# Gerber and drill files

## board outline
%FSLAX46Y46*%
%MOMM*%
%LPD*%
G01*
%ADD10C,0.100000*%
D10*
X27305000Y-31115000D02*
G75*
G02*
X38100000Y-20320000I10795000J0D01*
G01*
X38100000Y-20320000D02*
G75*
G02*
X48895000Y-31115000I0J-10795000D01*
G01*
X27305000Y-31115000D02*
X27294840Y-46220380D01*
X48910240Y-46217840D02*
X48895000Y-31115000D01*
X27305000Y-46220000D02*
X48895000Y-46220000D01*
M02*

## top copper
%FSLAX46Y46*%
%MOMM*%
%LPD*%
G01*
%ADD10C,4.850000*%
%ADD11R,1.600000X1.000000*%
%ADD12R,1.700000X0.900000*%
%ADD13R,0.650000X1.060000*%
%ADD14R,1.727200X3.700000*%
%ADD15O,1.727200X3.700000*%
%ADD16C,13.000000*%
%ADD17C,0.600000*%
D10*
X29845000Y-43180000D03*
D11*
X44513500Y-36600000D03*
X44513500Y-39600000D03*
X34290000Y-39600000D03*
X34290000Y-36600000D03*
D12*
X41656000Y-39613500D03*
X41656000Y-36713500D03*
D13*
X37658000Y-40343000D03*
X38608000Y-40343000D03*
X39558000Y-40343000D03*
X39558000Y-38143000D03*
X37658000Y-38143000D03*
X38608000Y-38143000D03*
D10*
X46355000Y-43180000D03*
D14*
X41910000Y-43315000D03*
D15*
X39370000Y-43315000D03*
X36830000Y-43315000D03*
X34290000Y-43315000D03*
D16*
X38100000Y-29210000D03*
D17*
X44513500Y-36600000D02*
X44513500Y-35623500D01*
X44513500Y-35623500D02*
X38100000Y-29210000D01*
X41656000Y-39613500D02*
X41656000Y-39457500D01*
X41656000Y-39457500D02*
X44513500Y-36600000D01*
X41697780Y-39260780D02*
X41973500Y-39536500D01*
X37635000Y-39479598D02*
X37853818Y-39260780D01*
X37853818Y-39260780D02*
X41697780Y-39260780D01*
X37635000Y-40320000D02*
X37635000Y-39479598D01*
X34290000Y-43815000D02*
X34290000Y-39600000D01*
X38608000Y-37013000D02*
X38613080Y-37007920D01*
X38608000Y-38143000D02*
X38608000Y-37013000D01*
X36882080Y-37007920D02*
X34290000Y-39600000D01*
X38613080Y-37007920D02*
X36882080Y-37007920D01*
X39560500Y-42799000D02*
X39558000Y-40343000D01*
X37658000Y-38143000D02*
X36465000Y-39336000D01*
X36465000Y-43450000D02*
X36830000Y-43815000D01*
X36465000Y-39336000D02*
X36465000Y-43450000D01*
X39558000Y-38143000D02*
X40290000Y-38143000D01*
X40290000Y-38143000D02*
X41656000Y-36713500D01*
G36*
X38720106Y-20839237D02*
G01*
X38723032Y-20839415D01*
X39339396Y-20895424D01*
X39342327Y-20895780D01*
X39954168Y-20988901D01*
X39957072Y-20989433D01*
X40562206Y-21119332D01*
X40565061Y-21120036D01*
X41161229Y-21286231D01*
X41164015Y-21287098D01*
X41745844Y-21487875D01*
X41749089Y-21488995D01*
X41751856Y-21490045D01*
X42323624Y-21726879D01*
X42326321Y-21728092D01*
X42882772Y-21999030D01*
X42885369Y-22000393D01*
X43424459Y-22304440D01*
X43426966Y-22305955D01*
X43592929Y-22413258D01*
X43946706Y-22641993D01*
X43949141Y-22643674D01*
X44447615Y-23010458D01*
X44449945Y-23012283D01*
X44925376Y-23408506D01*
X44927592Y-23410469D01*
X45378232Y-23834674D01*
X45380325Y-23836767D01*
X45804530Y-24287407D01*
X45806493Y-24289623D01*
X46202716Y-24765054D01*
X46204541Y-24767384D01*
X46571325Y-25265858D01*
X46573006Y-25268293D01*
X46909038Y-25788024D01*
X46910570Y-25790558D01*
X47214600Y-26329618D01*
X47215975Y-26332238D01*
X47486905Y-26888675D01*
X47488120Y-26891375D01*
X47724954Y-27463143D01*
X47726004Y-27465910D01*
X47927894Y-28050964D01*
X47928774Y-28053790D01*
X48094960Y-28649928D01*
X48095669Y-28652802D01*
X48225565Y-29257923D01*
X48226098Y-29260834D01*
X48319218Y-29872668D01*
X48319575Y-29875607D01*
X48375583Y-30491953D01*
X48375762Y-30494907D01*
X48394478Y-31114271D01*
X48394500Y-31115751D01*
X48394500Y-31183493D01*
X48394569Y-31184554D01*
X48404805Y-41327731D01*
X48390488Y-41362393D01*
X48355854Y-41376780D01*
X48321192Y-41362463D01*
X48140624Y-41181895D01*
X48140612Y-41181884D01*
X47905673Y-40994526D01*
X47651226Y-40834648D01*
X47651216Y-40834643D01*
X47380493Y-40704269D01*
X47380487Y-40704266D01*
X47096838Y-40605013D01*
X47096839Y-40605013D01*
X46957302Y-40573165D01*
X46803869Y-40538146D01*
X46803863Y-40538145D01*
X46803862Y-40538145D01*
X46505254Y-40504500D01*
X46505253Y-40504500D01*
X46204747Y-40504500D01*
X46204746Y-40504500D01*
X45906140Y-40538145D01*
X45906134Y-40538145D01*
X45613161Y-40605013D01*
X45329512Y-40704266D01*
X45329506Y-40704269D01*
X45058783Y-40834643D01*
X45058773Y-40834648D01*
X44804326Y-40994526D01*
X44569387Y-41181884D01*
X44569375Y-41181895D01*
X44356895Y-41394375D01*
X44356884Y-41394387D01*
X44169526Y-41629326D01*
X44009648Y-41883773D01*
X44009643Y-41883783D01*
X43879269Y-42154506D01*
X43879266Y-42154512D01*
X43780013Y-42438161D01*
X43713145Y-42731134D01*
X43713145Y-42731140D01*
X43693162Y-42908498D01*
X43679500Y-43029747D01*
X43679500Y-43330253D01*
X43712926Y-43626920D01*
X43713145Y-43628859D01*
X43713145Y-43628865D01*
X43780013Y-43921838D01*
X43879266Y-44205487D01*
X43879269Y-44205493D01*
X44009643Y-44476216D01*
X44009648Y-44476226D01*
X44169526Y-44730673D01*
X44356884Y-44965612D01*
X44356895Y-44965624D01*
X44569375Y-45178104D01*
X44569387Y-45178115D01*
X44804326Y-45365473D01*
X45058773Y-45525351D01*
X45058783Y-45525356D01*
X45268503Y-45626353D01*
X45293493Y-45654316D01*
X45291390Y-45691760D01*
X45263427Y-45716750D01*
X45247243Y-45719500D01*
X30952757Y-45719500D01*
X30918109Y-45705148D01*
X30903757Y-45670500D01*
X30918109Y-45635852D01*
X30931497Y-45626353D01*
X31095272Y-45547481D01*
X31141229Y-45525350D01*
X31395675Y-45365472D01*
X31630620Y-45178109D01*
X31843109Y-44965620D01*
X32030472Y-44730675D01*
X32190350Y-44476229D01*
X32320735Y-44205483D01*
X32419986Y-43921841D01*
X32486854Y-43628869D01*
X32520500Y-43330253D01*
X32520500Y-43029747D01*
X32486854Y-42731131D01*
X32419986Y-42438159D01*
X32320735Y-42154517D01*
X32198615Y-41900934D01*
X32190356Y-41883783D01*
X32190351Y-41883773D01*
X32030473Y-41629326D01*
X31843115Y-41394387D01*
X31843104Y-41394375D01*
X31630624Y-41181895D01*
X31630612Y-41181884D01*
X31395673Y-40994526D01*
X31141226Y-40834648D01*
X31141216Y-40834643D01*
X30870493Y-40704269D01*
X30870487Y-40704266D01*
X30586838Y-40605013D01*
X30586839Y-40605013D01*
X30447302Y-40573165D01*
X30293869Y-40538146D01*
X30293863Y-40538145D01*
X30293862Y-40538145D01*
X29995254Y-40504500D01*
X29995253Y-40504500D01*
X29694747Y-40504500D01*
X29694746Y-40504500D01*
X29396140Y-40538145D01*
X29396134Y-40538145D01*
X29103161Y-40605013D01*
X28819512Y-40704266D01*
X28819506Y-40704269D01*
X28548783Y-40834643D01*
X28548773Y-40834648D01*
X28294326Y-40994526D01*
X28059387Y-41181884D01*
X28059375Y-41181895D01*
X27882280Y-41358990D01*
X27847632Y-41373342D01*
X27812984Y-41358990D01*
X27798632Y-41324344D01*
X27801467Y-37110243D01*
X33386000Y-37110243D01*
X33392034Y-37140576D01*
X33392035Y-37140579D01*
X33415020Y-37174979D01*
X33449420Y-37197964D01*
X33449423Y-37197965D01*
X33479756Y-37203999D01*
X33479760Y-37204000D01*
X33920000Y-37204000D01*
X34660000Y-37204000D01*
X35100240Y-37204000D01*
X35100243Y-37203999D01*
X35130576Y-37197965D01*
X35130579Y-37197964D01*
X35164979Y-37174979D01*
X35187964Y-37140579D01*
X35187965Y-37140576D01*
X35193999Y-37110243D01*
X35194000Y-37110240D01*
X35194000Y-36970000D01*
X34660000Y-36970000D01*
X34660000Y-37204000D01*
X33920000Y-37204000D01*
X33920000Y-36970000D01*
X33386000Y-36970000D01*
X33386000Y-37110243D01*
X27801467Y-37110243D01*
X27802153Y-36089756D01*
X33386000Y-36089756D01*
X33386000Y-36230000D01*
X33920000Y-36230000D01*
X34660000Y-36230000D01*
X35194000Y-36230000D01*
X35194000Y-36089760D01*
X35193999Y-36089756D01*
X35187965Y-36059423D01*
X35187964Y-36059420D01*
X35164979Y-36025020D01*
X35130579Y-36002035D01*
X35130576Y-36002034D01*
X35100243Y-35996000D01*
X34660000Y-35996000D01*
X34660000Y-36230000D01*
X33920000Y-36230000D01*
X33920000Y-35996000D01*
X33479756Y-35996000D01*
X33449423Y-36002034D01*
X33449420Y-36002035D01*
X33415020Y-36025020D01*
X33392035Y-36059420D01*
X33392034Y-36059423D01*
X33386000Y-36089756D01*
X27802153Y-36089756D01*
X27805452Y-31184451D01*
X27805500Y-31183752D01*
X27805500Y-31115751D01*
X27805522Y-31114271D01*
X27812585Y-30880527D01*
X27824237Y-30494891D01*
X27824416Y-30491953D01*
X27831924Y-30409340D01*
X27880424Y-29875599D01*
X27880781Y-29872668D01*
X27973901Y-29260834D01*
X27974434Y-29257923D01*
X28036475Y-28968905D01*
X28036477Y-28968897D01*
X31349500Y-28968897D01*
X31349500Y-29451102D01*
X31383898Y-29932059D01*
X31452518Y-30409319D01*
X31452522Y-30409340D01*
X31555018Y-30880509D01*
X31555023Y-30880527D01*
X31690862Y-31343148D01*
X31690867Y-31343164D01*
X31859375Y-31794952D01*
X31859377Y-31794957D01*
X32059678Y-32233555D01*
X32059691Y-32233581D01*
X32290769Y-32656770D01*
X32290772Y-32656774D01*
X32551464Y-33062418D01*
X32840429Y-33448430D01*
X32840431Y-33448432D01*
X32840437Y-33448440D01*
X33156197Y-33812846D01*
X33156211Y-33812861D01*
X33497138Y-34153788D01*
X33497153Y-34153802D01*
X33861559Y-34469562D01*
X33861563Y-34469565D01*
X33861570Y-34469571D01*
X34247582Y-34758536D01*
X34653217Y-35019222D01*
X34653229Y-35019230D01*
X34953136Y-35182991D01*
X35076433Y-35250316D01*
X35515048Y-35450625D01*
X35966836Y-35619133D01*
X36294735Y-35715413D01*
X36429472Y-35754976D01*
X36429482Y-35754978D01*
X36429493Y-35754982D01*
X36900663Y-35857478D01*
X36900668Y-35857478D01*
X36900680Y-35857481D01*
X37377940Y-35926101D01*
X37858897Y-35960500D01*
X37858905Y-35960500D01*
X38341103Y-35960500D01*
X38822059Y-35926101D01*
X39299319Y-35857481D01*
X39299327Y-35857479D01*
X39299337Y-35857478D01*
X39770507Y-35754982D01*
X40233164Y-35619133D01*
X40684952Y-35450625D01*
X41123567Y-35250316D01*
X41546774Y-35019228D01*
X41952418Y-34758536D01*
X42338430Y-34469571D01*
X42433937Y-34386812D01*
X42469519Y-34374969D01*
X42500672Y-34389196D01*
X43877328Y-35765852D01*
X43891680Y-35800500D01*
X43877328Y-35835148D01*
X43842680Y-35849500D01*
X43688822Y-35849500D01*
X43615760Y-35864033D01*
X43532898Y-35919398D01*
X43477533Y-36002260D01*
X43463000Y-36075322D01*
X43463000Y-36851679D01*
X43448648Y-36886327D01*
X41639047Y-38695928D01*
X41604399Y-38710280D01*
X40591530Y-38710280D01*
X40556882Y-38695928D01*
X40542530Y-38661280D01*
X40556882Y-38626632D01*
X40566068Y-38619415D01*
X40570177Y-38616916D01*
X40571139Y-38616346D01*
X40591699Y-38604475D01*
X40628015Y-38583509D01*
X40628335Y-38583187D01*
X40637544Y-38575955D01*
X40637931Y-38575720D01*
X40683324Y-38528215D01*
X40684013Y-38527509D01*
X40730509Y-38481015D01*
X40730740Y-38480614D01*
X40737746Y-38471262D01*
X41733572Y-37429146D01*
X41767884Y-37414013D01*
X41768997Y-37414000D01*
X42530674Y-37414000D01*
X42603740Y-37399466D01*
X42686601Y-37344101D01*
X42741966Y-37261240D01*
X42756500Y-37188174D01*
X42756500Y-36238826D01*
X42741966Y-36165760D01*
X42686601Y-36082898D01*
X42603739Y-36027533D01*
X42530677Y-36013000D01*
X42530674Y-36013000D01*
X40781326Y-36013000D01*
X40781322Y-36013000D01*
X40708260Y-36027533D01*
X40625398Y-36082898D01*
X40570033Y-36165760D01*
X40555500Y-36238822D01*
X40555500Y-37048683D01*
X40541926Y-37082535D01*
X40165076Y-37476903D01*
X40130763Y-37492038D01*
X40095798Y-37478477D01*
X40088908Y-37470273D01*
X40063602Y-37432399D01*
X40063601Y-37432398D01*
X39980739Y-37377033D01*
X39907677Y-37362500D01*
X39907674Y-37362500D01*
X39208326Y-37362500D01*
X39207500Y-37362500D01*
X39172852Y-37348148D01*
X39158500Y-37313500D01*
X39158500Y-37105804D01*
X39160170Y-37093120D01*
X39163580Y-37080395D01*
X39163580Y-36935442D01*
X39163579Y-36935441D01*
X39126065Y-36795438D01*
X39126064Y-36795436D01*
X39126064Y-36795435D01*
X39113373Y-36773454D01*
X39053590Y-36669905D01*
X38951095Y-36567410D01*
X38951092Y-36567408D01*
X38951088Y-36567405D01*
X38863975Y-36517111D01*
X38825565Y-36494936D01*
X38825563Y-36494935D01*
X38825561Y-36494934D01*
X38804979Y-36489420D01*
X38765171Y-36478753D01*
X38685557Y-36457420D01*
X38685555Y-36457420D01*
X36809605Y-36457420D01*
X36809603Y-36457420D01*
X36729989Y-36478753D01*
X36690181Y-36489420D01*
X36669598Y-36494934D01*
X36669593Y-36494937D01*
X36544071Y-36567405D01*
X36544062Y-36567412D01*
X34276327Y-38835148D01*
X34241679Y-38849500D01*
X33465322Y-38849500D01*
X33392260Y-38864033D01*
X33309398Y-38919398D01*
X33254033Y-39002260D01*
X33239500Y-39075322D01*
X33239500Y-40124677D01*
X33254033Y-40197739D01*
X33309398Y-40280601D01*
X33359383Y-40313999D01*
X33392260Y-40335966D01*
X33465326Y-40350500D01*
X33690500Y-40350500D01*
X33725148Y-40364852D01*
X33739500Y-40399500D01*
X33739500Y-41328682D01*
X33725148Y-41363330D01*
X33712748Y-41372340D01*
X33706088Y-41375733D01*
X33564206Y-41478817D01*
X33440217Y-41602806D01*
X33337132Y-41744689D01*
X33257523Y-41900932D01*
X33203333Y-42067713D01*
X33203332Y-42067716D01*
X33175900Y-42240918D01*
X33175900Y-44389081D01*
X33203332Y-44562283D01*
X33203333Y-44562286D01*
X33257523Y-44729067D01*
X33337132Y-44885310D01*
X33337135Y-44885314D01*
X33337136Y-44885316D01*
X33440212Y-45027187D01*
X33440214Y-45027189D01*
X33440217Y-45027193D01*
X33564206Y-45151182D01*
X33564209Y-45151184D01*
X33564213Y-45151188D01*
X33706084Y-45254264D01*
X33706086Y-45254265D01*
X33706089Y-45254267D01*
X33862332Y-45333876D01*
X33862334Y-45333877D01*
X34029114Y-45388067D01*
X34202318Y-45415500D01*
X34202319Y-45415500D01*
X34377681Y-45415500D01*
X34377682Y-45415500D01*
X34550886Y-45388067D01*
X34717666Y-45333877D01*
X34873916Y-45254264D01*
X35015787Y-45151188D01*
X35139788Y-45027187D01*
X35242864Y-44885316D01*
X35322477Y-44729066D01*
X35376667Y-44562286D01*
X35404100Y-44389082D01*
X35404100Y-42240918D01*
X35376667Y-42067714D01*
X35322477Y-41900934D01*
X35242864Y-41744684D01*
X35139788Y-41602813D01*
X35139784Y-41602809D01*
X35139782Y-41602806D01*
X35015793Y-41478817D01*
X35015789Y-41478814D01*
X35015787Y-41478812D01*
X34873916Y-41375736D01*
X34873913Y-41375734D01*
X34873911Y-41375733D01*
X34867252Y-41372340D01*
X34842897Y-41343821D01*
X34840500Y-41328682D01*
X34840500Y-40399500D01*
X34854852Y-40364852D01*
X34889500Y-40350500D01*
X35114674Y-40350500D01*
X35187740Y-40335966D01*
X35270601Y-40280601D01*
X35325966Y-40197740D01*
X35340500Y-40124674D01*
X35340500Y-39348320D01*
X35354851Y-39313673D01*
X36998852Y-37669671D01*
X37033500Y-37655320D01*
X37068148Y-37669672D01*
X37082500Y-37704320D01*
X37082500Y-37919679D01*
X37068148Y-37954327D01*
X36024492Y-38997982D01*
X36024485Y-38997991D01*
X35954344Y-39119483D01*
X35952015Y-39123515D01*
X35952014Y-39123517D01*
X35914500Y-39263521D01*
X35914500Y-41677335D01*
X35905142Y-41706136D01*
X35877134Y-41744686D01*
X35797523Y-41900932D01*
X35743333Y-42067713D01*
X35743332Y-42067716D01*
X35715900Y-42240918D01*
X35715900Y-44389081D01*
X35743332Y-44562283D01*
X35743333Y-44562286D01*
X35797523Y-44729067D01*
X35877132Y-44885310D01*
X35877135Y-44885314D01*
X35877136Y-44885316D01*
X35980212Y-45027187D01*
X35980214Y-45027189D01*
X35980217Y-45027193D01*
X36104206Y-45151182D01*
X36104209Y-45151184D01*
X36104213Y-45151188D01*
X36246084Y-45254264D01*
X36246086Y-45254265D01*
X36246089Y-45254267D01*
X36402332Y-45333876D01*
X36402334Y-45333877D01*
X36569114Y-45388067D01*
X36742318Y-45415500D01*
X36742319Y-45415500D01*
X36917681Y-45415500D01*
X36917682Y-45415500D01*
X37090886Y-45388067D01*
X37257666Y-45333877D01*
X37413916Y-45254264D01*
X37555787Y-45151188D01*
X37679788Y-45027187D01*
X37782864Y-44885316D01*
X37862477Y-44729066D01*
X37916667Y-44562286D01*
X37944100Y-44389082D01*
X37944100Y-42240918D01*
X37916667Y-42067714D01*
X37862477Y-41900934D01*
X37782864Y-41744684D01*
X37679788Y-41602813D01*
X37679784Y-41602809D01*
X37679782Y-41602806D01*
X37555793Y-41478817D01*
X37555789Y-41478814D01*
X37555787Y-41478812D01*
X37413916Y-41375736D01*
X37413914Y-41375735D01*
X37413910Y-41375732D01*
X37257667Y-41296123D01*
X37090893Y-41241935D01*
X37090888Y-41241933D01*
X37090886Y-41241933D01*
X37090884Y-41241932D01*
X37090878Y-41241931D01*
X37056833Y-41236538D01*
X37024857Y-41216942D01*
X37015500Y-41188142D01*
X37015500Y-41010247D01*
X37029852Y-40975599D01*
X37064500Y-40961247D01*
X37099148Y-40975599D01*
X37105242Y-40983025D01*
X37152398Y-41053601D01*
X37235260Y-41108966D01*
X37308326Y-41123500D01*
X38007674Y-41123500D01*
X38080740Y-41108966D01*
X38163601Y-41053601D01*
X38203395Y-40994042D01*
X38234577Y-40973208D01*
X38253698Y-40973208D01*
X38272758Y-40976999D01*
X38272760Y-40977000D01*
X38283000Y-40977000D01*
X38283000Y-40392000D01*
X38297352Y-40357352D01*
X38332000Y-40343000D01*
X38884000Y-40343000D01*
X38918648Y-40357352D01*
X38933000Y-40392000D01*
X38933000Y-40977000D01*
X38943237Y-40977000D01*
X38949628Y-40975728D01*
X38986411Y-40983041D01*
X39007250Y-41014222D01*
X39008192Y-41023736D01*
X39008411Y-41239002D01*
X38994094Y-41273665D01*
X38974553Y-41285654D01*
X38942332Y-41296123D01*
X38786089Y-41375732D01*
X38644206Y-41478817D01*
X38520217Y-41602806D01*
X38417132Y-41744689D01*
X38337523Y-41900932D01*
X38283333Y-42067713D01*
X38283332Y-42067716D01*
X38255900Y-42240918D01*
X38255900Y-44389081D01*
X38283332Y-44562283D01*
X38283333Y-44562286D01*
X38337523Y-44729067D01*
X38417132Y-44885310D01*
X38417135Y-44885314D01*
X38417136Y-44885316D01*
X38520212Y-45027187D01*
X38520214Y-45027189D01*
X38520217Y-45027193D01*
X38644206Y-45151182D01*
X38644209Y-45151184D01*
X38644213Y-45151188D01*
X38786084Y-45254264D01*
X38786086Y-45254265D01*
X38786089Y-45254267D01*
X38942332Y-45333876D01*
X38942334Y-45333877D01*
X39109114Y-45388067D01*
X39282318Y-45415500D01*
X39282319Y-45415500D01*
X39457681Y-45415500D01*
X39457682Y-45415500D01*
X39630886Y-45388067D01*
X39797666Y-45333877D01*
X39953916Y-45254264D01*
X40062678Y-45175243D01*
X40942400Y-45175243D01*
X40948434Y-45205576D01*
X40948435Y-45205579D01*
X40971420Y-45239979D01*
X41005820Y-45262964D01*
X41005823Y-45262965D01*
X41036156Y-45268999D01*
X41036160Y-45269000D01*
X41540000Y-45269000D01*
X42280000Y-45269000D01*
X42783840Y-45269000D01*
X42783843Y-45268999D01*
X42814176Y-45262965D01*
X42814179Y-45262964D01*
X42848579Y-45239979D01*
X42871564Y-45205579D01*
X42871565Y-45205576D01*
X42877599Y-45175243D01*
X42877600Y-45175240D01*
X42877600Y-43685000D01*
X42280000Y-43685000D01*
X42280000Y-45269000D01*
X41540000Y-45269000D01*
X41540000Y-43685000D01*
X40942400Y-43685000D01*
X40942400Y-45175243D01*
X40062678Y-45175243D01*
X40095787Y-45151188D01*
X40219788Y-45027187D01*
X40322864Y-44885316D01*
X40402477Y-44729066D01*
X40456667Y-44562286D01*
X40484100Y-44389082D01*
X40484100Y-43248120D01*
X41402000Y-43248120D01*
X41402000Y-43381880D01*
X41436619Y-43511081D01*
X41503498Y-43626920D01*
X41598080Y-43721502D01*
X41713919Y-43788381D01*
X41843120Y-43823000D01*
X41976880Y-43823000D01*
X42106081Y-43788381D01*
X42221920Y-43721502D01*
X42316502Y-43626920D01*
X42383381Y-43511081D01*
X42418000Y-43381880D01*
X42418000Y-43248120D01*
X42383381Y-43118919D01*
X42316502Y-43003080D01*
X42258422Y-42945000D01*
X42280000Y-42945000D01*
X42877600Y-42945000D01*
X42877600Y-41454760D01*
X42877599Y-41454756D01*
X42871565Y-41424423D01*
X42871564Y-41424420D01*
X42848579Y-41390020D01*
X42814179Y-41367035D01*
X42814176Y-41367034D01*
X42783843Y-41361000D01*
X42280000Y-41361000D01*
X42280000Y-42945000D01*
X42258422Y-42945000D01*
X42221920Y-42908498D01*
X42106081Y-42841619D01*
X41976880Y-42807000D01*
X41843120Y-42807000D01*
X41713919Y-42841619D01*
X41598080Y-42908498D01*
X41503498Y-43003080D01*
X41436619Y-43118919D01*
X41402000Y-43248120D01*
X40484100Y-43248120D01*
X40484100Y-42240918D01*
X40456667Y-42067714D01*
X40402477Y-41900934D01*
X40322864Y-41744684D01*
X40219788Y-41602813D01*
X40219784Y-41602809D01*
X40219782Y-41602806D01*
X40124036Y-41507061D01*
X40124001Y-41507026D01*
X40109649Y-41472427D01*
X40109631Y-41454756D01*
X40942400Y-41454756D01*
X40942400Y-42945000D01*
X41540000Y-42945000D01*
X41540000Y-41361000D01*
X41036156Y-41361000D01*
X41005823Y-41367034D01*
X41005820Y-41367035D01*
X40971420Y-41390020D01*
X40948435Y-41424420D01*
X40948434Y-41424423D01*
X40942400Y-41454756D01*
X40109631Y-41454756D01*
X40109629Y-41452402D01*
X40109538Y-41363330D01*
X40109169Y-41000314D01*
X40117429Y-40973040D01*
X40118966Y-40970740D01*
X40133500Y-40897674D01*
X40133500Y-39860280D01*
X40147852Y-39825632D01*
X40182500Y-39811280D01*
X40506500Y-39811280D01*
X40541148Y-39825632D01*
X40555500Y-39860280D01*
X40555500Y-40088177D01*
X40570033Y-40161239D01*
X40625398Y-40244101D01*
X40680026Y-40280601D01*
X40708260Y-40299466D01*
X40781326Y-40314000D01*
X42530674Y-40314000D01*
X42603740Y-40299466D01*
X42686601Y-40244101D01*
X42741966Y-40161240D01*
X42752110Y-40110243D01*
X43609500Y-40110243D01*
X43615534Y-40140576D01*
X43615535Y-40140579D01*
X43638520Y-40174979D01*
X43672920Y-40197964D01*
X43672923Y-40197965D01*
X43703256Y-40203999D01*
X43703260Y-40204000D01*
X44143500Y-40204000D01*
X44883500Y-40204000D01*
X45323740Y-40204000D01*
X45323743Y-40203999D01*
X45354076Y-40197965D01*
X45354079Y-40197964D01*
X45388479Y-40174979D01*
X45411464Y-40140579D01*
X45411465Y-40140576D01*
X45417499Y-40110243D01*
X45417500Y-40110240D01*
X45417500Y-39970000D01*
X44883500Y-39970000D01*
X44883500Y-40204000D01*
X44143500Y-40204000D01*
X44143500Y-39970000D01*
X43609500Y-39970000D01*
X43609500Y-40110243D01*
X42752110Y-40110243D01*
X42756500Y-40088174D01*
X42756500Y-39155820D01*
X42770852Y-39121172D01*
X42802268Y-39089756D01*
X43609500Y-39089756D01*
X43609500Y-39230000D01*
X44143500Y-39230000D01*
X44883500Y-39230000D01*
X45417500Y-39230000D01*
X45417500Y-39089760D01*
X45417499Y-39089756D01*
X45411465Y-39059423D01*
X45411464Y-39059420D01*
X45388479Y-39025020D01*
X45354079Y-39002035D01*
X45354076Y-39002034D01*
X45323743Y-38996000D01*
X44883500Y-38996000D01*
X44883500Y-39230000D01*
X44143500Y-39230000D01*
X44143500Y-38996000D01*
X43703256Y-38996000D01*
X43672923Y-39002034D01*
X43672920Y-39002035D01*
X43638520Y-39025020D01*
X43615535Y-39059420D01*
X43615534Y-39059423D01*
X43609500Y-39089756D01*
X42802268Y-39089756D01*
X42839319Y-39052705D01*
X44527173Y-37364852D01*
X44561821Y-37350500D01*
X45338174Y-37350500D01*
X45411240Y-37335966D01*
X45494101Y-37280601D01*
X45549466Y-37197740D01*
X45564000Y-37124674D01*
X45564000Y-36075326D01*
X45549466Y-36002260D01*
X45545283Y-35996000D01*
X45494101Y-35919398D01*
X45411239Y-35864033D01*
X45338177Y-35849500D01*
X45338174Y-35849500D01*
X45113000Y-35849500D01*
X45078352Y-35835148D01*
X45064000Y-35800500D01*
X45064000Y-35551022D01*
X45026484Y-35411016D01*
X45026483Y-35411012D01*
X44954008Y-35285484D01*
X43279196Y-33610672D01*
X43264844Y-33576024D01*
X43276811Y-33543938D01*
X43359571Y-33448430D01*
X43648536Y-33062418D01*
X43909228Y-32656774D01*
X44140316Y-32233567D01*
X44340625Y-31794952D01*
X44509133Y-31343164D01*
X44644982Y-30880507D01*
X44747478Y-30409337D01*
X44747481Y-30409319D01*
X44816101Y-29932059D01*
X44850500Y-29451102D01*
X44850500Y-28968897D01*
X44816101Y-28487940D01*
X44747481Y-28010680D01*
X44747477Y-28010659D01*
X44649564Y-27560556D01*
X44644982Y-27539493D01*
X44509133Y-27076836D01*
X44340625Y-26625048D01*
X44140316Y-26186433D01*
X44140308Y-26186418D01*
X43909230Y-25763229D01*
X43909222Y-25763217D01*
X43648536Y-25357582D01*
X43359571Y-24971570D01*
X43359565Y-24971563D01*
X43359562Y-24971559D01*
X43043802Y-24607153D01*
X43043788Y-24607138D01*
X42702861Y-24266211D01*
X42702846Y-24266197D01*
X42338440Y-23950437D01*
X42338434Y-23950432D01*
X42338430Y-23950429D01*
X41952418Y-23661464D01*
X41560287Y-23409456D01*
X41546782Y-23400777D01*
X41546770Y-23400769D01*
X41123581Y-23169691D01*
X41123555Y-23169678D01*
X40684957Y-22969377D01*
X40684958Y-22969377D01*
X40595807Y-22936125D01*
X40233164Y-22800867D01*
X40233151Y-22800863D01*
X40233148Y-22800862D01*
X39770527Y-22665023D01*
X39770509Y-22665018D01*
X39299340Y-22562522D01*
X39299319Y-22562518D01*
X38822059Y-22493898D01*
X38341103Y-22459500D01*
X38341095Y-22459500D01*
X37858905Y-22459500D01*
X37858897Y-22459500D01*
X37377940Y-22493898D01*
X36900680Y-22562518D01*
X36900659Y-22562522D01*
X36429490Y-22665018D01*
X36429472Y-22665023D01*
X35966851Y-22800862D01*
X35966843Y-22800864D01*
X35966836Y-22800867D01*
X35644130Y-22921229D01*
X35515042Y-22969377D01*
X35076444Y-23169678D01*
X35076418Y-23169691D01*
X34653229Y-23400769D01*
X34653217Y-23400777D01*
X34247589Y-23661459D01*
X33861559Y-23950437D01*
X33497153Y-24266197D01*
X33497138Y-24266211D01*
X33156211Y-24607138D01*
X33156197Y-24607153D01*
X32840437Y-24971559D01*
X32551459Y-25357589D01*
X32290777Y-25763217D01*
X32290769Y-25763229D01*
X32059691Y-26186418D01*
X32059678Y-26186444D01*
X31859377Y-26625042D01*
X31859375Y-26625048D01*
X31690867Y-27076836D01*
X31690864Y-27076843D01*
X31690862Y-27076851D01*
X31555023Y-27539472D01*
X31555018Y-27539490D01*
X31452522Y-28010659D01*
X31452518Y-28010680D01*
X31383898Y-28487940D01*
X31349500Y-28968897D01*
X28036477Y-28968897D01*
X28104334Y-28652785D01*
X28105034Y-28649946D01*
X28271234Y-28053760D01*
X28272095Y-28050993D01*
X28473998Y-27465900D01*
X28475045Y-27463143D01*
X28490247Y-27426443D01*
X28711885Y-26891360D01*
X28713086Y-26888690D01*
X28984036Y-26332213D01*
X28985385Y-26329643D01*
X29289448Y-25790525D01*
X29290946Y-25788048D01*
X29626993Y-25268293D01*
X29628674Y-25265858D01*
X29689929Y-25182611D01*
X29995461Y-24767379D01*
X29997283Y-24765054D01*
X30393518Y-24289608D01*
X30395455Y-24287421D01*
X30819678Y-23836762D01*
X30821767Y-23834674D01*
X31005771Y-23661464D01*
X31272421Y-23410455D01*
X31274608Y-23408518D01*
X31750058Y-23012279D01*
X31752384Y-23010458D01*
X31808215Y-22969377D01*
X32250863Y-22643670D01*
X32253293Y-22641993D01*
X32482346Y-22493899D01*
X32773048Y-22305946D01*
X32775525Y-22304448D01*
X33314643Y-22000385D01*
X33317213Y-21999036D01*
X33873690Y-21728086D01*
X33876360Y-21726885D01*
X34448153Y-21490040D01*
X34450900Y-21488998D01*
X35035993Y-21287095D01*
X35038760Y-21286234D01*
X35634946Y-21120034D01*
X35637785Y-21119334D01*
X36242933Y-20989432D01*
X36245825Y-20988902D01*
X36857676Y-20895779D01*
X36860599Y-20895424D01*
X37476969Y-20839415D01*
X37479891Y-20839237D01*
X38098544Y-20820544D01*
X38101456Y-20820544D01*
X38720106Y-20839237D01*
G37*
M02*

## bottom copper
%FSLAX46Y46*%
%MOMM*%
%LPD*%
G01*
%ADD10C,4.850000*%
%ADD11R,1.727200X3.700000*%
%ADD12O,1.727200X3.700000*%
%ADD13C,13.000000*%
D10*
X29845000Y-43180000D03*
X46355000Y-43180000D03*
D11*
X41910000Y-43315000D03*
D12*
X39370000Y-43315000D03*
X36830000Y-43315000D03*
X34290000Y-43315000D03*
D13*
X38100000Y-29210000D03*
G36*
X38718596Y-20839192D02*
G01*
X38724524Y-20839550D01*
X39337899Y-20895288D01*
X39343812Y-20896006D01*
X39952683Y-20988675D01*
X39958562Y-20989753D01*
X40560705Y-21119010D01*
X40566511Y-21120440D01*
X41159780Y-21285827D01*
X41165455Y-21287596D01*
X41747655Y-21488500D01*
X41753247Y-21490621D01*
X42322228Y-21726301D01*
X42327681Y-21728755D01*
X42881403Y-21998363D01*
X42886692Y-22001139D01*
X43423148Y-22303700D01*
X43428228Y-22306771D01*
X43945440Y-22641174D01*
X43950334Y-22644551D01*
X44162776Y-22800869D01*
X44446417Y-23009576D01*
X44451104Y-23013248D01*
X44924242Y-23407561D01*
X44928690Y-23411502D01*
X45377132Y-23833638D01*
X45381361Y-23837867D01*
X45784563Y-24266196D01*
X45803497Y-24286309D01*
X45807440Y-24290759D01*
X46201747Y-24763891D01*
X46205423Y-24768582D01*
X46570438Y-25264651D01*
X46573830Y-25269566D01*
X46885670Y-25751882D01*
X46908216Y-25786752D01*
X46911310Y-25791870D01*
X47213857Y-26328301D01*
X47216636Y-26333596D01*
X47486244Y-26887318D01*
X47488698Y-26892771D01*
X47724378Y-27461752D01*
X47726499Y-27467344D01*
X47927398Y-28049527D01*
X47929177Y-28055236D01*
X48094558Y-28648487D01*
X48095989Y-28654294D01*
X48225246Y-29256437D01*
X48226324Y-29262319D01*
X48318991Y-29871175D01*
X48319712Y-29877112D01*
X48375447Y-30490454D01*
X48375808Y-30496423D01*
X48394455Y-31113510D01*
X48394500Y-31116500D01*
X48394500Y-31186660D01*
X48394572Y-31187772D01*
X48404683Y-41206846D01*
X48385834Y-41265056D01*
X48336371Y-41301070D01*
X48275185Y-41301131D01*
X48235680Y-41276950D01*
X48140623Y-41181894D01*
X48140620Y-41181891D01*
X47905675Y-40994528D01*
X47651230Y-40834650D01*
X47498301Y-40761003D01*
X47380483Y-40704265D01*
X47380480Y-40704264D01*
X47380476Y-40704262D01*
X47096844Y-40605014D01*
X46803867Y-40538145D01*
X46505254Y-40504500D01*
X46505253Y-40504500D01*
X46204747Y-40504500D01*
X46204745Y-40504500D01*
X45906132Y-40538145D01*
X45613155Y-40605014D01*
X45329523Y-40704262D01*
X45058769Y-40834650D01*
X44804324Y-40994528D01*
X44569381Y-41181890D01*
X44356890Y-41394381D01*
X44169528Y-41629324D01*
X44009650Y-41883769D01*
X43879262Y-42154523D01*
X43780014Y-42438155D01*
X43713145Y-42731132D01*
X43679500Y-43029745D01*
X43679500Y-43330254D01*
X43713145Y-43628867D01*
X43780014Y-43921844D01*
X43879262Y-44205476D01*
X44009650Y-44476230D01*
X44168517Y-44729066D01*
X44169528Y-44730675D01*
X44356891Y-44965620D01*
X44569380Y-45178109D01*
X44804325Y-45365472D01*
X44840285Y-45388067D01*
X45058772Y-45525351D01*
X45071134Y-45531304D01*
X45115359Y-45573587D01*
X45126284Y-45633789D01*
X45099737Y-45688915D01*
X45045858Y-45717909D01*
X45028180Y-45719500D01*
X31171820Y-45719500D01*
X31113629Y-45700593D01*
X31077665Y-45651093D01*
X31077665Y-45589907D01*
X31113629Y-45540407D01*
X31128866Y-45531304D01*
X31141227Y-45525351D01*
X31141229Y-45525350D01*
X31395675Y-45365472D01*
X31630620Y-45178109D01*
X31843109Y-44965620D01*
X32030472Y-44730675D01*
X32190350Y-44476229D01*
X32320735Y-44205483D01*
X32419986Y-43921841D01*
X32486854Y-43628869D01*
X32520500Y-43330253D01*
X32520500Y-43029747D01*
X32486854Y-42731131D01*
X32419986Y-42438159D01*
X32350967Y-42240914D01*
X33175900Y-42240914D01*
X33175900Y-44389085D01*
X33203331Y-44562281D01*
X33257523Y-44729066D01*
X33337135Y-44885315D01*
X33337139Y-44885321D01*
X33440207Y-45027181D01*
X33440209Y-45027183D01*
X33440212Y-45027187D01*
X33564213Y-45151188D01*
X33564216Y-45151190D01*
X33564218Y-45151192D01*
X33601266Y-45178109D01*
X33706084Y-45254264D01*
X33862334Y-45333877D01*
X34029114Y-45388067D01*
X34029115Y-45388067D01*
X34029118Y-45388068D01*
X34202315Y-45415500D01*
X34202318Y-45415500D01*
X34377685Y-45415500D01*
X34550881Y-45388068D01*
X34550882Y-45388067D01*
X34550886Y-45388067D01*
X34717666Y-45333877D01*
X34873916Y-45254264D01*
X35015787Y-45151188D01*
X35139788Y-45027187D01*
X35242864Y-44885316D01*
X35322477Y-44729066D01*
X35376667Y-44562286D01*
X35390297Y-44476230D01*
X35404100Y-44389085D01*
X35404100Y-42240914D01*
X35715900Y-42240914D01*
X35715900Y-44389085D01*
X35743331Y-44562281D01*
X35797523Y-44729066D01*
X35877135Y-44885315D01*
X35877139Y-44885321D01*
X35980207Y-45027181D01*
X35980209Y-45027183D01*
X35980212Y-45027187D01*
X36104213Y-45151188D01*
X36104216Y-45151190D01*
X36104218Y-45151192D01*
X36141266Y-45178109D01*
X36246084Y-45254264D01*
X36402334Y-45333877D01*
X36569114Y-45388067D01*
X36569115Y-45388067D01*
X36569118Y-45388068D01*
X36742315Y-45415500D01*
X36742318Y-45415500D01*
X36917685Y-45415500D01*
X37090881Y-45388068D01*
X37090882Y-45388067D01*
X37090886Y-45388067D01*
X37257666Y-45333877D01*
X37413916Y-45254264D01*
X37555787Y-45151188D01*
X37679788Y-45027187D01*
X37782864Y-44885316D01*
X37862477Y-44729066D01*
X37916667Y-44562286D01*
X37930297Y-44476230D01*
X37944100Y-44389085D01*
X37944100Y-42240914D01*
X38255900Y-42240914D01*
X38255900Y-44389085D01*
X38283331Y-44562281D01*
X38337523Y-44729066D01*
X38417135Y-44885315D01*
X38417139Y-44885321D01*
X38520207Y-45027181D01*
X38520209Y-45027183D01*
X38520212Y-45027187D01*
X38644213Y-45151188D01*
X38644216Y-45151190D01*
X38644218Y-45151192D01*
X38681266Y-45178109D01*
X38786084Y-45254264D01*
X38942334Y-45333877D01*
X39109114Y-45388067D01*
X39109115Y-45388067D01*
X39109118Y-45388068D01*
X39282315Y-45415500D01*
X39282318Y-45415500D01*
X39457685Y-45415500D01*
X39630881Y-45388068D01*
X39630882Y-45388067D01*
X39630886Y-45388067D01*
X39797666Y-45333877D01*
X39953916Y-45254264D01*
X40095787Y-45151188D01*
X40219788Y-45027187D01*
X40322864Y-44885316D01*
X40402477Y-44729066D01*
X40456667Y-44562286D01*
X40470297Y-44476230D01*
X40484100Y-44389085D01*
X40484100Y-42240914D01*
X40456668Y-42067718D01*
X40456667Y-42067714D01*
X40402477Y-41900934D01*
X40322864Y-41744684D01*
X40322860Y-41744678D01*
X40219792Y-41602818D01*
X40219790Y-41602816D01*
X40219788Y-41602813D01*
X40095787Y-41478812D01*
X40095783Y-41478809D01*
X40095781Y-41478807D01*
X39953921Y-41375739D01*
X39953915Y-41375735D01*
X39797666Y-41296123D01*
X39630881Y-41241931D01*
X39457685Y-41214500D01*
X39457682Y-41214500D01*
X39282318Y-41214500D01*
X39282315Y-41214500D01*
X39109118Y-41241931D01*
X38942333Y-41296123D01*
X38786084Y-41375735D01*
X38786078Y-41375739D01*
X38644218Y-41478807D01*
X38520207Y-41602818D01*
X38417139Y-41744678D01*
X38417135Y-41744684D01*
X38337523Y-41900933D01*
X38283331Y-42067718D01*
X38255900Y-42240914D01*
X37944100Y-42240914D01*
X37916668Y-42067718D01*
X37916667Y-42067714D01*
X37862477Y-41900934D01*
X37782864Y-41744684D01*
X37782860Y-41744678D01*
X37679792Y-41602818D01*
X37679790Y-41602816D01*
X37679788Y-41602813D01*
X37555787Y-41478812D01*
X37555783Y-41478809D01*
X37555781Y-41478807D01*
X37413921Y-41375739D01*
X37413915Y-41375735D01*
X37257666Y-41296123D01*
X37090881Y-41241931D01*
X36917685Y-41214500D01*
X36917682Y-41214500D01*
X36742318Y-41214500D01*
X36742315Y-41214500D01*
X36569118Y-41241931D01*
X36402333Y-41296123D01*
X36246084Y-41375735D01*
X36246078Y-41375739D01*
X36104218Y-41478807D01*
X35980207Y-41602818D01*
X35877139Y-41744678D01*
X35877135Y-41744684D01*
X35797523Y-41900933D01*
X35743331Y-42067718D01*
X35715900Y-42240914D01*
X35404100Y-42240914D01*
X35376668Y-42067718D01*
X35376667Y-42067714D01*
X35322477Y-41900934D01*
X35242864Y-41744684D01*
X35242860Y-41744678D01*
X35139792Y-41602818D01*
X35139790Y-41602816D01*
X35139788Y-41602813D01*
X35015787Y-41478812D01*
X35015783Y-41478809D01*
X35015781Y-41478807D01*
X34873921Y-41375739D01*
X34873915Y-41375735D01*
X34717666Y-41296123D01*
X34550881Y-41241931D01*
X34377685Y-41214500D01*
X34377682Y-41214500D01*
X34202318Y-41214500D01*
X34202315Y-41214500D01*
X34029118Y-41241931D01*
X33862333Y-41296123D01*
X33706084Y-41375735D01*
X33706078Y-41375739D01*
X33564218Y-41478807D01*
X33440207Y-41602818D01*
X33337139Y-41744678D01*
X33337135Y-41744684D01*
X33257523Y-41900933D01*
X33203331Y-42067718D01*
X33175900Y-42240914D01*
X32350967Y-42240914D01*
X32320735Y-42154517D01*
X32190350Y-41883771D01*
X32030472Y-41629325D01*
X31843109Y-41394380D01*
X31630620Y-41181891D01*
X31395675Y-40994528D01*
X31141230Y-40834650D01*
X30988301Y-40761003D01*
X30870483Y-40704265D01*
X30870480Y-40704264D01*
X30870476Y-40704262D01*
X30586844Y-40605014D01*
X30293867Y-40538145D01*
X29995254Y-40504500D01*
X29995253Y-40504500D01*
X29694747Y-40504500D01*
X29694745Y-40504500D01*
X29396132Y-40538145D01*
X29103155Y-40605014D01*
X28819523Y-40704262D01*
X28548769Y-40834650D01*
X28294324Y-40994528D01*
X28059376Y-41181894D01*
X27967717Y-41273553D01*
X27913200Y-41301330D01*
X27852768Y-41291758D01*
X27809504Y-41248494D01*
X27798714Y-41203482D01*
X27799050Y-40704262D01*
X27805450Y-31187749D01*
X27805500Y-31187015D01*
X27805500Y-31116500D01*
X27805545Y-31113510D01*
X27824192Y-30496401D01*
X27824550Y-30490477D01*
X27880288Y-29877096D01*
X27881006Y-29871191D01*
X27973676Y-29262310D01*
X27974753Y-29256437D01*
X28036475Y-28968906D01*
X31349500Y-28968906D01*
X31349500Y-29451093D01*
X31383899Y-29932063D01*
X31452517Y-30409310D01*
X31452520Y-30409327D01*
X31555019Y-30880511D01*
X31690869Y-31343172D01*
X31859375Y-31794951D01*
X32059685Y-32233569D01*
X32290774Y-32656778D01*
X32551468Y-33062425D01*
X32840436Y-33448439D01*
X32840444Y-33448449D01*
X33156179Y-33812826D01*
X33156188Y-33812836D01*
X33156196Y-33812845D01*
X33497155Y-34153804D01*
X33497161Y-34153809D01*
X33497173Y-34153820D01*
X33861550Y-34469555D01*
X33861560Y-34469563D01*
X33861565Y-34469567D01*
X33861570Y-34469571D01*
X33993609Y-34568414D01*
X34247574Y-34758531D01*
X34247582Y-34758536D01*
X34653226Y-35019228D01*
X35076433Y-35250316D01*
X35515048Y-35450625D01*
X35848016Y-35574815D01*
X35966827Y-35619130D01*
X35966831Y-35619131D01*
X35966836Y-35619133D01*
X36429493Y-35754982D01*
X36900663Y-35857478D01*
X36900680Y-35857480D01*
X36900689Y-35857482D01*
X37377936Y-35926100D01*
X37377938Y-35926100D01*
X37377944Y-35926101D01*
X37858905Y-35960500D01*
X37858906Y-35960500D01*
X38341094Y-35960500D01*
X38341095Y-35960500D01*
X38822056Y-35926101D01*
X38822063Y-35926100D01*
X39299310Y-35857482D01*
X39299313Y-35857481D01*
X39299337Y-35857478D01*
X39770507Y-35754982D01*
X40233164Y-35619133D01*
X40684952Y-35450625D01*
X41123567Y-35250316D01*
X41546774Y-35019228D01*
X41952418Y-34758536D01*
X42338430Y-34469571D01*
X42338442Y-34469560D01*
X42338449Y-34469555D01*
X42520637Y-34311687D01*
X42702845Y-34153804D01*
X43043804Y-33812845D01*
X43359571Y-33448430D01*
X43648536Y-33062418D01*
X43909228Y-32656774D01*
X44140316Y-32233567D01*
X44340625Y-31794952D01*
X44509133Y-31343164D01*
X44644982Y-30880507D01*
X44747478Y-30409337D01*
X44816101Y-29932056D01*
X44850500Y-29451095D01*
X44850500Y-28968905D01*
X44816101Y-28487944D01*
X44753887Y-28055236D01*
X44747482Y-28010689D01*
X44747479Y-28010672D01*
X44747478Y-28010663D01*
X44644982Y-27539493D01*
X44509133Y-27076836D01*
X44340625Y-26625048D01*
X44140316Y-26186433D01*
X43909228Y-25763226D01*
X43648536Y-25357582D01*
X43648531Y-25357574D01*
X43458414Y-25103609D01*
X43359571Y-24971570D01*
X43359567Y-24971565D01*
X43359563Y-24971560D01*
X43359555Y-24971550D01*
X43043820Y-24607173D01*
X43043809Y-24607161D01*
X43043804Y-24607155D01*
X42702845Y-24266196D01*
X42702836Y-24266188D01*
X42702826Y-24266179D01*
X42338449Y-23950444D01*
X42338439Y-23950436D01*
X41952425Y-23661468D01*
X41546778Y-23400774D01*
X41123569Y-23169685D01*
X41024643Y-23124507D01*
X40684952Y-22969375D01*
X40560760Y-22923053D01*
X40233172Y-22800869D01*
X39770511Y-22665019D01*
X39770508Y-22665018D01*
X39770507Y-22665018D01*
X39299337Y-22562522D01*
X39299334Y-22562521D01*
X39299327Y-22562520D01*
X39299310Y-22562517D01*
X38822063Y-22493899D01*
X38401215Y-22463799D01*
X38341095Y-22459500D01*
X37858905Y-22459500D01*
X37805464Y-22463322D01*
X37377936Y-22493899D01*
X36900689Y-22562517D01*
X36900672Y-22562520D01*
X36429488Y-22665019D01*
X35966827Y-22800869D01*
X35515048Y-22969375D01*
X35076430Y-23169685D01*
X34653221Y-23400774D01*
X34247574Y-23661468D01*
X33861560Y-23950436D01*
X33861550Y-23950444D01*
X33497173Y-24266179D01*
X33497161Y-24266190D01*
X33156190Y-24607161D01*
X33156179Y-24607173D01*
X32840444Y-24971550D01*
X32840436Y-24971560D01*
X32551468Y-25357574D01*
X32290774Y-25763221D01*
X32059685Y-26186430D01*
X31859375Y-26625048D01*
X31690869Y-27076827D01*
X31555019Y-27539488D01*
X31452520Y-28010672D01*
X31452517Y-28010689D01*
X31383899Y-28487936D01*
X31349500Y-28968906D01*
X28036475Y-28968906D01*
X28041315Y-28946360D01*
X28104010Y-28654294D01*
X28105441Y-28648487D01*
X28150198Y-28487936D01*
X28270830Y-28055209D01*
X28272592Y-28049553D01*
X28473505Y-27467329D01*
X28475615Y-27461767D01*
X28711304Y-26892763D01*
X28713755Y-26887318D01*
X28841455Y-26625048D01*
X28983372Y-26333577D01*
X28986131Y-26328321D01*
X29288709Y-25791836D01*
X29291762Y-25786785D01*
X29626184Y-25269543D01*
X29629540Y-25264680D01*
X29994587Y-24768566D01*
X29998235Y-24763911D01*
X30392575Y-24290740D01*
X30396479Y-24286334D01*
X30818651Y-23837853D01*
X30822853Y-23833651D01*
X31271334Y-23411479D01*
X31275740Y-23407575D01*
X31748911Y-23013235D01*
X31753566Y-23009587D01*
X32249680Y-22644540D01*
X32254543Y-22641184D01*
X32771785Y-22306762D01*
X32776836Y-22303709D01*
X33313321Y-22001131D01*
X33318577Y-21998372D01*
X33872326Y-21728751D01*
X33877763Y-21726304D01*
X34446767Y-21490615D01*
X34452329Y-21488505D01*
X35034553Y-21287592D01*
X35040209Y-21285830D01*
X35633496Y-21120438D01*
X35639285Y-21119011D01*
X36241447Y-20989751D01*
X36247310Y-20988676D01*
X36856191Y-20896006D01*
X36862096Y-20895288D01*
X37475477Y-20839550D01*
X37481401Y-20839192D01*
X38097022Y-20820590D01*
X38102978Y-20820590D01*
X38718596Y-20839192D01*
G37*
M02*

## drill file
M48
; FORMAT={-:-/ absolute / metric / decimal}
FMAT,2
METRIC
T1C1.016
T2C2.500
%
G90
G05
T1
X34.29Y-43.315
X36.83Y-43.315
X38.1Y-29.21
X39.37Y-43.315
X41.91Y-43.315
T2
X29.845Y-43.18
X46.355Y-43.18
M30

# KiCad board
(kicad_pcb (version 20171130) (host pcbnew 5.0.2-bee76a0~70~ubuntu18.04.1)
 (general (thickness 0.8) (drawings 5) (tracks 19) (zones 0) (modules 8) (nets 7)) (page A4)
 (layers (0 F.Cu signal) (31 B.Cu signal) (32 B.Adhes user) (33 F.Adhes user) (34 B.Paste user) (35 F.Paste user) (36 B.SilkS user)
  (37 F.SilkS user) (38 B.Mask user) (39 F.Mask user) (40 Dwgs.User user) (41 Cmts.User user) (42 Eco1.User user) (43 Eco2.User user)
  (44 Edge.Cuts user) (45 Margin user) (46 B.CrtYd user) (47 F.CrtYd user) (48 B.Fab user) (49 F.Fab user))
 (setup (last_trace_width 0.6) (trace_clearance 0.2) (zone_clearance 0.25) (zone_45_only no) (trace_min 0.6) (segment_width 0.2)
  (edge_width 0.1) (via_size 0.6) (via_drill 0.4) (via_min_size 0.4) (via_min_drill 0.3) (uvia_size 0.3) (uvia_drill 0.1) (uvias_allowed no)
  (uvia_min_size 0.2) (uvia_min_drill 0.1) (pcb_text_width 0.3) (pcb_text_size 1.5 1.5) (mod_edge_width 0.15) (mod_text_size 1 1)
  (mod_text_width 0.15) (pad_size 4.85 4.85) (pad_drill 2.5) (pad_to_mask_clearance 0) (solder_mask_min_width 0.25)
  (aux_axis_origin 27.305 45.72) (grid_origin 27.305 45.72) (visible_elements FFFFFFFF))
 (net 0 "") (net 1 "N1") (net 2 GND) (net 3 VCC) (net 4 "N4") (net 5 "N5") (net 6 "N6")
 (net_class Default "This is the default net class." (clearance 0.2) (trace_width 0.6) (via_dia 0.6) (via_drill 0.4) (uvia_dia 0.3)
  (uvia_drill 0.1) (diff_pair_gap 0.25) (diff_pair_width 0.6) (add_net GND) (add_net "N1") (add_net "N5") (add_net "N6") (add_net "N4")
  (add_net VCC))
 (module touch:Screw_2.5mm (layer F.Cu) (at 29.845 43.18 90)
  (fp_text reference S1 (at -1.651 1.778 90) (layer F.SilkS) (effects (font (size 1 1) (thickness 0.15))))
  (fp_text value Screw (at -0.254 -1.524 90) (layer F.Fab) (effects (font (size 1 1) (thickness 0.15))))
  (pad 1 thru_hole circle (at 0 0 90) (size 4.85 4.85) (drill 2.5) (layers *.Cu *.Mask F.SilkS)))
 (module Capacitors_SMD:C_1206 (layer F.Cu) (at 44.5135 38.1 270)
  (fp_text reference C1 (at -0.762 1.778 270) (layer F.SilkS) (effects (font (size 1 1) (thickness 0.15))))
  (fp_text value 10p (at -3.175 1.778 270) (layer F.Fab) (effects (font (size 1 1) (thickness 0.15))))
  (pad 1 smd rect (at -1.5 0 270) (size 1 1.6) (layers F.Cu F.Paste F.Mask) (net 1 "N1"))
  (pad 2 smd rect (at 1.5 0 270) (size 1 1.6) (layers F.Cu F.Paste F.Mask) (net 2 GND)))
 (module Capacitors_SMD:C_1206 (layer F.Cu) (at 34.29 38.1 90)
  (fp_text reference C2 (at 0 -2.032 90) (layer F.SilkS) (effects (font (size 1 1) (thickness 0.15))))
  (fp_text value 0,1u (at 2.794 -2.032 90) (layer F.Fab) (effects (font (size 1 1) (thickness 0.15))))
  (pad 1 smd rect (at -1.5 0 90) (size 1 1.6) (layers F.Cu F.Paste F.Mask) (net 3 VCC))
  (pad 2 smd rect (at 1.5 0 90) (size 1 1.6) (layers F.Cu F.Paste F.Mask) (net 2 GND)))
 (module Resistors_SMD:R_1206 (layer F.Cu) (at 41.656 38.1635 90)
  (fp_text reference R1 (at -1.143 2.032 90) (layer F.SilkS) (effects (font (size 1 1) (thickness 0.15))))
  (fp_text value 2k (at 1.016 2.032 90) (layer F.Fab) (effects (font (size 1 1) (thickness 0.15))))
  (pad 1 smd rect (at -1.45 0 90) (size 0.9 1.7) (layers F.Cu F.Paste F.Mask) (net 1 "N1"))
  (pad 2 smd rect (at 1.45 0 90) (size 0.9 1.7) (layers F.Cu F.Paste F.Mask) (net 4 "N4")))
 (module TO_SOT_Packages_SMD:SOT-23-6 (layer F.Cu) (at 38.608 39.243 90)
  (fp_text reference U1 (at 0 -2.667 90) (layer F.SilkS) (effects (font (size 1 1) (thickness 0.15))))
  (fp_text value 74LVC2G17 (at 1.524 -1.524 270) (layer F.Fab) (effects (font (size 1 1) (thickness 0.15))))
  (pad 1 smd rect (at -1.1 -0.95 90) (size 1.06 0.65) (layers F.Cu F.Paste F.Mask) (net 1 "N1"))
  (pad 2 smd rect (at -1.1 0 90) (size 1.06 0.65) (layers F.Cu F.Paste F.Mask) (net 2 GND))
  (pad 3 smd rect (at -1.1 0.95 90) (size 1.06 0.65) (layers F.Cu F.Paste F.Mask) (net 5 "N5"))
  (pad 4 smd rect (at 1.1 0.95 90) (size 1.06 0.65) (layers F.Cu F.Paste F.Mask) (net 4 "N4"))
  (pad 6 smd rect (at 1.1 -0.95 90) (size 1.06 0.65) (layers F.Cu F.Paste F.Mask) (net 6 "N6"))
  (pad 5 smd rect (at 1.1 0 90) (size 1.06 0.65) (layers F.Cu F.Paste F.Mask) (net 3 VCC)))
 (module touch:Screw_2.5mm (layer F.Cu) (at 46.355 43.18 90)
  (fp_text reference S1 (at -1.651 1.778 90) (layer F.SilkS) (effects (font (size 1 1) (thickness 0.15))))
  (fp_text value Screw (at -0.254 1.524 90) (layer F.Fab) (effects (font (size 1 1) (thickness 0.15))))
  (pad 1 thru_hole circle (at 0 0 90) (size 4.85 4.85) (drill 2.5) (layers *.Cu *.Mask F.SilkS)))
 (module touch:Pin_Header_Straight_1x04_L (layer F.Cu) (at 41.91 43.315 270)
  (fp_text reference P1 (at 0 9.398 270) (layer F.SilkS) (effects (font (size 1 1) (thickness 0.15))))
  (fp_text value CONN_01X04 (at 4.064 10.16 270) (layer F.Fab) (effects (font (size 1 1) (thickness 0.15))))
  (pad 1 thru_hole rect (at 0 0 270) (size 3.7 1.7272) (drill 1.016) (layers *.Cu *.Mask F.SilkS) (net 2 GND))
  (pad 2 thru_hole oval (at 0 2.54 270) (size 3.7 1.7272) (drill 1.016) (layers *.Cu *.Mask F.SilkS) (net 5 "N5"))
  (pad 3 thru_hole oval (at 0 5.08 270) (size 3.7 1.7272) (drill 1.016) (layers *.Cu *.Mask F.SilkS) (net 6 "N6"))
  (pad 4 thru_hole oval (at 0 7.62 270) (size 3.7 1.7272) (drill 1.016) (layers *.Cu *.Mask F.SilkS) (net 3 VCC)))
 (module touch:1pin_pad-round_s (layer F.Cu) (at 38.1 29.21 90)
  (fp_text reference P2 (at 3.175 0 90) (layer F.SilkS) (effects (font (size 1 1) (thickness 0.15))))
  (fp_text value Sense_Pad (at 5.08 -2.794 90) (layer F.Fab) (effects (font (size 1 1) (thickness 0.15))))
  (pad 1 thru_hole circle (at 0 0 90) (size 13 13) (drill 1.016) (layers *.Cu *.Mask F.SilkS) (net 1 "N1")))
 (gr_arc (start 38.1 31.115) (end 27.305 31.115) (angle 90) (layer Edge.Cuts) (width 0.1))
 (gr_arc (start 38.1 31.115) (end 38.1 20.32) (angle 90) (layer Edge.Cuts) (width 0.1))
 (gr_line (start 27.305 31.115) (end 27.29484 46.22038) (angle 90) (layer Edge.Cuts) (width 0.1))
 (gr_line (start 48.91024 46.21784) (end 48.895 31.115) (angle 90) (layer Edge.Cuts) (width 0.1))
 (gr_line (start 27.305 46.22) (end 48.895 46.22) (angle 90) (layer Edge.Cuts) (width 0.1))
 (segment (start 44.5135 36.6) (end 44.5135 35.6235) (width 0.6) (layer F.Cu) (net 1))
 (segment (start 44.5135 35.6235) (end 38.1 29.21) (width 0.6) (layer F.Cu) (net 1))
 (segment (start 41.656 39.6135) (end 41.656 39.4575) (width 0.6) (layer F.Cu) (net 1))
 (segment (start 41.656 39.4575) (end 44.5135 36.6) (width 0.6) (layer F.Cu) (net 1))
 (segment (start 41.69778 39.26078) (end 41.9735 39.5365) (width 0.6) (layer F.Cu) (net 1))
 (segment (start 37.635 39.479598) (end 37.853818 39.26078) (width 0.6) (layer F.Cu) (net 1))
 (segment (start 37.853818 39.26078) (end 41.69778 39.26078) (width 0.6) (layer F.Cu) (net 1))
 (segment (start 37.635 40.32) (end 37.635 39.479598) (width 0.6) (layer F.Cu) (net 1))
 (segment (start 34.29 43.815) (end 34.29 39.6) (width 0.6) (layer F.Cu) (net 3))
 (segment (start 38.608 37.013) (end 38.61308 37.00792) (width 0.6) (layer F.Cu) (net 3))
 (segment (start 38.608 38.143) (end 38.608 37.013) (width 0.6) (layer F.Cu) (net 3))
 (segment (start 36.88208 37.00792) (end 34.29 39.6) (width 0.6) (layer F.Cu) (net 3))
 (segment (start 38.61308 37.00792) (end 36.88208 37.00792) (width 0.6) (layer F.Cu) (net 3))
 (segment (start 39.5605 42.799) (end 39.558 40.343) (width 0.6) (layer F.Cu) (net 5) (status 20))
 (segment (start 37.658 38.143) (end 36.465 39.336) (width 0.6) (layer F.Cu) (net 6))
 (segment (start 36.465 43.45) (end 36.83 43.815) (width 0.6) (layer F.Cu) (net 6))
 (segment (start 36.465 39.336) (end 36.465 43.45) (width 0.6) (layer F.Cu) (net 6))
 (segment (start 39.558 38.143) (end 40.29 38.143) (width 0.6) (layer F.Cu) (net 4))
 (segment (start 40.29 38.143) (end 41.656 36.7135) (width 0.6) (layer F.Cu) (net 4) (status 20))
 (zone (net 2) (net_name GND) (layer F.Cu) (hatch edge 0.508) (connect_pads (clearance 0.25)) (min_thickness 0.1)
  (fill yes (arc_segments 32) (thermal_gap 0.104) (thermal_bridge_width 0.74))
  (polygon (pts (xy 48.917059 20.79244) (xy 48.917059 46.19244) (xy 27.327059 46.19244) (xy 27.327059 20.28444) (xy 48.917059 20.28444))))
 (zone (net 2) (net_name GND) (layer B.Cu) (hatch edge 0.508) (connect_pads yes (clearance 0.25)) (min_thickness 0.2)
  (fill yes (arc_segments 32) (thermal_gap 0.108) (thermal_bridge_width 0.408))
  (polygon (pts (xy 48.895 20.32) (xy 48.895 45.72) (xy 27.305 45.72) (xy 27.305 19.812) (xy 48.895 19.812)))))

